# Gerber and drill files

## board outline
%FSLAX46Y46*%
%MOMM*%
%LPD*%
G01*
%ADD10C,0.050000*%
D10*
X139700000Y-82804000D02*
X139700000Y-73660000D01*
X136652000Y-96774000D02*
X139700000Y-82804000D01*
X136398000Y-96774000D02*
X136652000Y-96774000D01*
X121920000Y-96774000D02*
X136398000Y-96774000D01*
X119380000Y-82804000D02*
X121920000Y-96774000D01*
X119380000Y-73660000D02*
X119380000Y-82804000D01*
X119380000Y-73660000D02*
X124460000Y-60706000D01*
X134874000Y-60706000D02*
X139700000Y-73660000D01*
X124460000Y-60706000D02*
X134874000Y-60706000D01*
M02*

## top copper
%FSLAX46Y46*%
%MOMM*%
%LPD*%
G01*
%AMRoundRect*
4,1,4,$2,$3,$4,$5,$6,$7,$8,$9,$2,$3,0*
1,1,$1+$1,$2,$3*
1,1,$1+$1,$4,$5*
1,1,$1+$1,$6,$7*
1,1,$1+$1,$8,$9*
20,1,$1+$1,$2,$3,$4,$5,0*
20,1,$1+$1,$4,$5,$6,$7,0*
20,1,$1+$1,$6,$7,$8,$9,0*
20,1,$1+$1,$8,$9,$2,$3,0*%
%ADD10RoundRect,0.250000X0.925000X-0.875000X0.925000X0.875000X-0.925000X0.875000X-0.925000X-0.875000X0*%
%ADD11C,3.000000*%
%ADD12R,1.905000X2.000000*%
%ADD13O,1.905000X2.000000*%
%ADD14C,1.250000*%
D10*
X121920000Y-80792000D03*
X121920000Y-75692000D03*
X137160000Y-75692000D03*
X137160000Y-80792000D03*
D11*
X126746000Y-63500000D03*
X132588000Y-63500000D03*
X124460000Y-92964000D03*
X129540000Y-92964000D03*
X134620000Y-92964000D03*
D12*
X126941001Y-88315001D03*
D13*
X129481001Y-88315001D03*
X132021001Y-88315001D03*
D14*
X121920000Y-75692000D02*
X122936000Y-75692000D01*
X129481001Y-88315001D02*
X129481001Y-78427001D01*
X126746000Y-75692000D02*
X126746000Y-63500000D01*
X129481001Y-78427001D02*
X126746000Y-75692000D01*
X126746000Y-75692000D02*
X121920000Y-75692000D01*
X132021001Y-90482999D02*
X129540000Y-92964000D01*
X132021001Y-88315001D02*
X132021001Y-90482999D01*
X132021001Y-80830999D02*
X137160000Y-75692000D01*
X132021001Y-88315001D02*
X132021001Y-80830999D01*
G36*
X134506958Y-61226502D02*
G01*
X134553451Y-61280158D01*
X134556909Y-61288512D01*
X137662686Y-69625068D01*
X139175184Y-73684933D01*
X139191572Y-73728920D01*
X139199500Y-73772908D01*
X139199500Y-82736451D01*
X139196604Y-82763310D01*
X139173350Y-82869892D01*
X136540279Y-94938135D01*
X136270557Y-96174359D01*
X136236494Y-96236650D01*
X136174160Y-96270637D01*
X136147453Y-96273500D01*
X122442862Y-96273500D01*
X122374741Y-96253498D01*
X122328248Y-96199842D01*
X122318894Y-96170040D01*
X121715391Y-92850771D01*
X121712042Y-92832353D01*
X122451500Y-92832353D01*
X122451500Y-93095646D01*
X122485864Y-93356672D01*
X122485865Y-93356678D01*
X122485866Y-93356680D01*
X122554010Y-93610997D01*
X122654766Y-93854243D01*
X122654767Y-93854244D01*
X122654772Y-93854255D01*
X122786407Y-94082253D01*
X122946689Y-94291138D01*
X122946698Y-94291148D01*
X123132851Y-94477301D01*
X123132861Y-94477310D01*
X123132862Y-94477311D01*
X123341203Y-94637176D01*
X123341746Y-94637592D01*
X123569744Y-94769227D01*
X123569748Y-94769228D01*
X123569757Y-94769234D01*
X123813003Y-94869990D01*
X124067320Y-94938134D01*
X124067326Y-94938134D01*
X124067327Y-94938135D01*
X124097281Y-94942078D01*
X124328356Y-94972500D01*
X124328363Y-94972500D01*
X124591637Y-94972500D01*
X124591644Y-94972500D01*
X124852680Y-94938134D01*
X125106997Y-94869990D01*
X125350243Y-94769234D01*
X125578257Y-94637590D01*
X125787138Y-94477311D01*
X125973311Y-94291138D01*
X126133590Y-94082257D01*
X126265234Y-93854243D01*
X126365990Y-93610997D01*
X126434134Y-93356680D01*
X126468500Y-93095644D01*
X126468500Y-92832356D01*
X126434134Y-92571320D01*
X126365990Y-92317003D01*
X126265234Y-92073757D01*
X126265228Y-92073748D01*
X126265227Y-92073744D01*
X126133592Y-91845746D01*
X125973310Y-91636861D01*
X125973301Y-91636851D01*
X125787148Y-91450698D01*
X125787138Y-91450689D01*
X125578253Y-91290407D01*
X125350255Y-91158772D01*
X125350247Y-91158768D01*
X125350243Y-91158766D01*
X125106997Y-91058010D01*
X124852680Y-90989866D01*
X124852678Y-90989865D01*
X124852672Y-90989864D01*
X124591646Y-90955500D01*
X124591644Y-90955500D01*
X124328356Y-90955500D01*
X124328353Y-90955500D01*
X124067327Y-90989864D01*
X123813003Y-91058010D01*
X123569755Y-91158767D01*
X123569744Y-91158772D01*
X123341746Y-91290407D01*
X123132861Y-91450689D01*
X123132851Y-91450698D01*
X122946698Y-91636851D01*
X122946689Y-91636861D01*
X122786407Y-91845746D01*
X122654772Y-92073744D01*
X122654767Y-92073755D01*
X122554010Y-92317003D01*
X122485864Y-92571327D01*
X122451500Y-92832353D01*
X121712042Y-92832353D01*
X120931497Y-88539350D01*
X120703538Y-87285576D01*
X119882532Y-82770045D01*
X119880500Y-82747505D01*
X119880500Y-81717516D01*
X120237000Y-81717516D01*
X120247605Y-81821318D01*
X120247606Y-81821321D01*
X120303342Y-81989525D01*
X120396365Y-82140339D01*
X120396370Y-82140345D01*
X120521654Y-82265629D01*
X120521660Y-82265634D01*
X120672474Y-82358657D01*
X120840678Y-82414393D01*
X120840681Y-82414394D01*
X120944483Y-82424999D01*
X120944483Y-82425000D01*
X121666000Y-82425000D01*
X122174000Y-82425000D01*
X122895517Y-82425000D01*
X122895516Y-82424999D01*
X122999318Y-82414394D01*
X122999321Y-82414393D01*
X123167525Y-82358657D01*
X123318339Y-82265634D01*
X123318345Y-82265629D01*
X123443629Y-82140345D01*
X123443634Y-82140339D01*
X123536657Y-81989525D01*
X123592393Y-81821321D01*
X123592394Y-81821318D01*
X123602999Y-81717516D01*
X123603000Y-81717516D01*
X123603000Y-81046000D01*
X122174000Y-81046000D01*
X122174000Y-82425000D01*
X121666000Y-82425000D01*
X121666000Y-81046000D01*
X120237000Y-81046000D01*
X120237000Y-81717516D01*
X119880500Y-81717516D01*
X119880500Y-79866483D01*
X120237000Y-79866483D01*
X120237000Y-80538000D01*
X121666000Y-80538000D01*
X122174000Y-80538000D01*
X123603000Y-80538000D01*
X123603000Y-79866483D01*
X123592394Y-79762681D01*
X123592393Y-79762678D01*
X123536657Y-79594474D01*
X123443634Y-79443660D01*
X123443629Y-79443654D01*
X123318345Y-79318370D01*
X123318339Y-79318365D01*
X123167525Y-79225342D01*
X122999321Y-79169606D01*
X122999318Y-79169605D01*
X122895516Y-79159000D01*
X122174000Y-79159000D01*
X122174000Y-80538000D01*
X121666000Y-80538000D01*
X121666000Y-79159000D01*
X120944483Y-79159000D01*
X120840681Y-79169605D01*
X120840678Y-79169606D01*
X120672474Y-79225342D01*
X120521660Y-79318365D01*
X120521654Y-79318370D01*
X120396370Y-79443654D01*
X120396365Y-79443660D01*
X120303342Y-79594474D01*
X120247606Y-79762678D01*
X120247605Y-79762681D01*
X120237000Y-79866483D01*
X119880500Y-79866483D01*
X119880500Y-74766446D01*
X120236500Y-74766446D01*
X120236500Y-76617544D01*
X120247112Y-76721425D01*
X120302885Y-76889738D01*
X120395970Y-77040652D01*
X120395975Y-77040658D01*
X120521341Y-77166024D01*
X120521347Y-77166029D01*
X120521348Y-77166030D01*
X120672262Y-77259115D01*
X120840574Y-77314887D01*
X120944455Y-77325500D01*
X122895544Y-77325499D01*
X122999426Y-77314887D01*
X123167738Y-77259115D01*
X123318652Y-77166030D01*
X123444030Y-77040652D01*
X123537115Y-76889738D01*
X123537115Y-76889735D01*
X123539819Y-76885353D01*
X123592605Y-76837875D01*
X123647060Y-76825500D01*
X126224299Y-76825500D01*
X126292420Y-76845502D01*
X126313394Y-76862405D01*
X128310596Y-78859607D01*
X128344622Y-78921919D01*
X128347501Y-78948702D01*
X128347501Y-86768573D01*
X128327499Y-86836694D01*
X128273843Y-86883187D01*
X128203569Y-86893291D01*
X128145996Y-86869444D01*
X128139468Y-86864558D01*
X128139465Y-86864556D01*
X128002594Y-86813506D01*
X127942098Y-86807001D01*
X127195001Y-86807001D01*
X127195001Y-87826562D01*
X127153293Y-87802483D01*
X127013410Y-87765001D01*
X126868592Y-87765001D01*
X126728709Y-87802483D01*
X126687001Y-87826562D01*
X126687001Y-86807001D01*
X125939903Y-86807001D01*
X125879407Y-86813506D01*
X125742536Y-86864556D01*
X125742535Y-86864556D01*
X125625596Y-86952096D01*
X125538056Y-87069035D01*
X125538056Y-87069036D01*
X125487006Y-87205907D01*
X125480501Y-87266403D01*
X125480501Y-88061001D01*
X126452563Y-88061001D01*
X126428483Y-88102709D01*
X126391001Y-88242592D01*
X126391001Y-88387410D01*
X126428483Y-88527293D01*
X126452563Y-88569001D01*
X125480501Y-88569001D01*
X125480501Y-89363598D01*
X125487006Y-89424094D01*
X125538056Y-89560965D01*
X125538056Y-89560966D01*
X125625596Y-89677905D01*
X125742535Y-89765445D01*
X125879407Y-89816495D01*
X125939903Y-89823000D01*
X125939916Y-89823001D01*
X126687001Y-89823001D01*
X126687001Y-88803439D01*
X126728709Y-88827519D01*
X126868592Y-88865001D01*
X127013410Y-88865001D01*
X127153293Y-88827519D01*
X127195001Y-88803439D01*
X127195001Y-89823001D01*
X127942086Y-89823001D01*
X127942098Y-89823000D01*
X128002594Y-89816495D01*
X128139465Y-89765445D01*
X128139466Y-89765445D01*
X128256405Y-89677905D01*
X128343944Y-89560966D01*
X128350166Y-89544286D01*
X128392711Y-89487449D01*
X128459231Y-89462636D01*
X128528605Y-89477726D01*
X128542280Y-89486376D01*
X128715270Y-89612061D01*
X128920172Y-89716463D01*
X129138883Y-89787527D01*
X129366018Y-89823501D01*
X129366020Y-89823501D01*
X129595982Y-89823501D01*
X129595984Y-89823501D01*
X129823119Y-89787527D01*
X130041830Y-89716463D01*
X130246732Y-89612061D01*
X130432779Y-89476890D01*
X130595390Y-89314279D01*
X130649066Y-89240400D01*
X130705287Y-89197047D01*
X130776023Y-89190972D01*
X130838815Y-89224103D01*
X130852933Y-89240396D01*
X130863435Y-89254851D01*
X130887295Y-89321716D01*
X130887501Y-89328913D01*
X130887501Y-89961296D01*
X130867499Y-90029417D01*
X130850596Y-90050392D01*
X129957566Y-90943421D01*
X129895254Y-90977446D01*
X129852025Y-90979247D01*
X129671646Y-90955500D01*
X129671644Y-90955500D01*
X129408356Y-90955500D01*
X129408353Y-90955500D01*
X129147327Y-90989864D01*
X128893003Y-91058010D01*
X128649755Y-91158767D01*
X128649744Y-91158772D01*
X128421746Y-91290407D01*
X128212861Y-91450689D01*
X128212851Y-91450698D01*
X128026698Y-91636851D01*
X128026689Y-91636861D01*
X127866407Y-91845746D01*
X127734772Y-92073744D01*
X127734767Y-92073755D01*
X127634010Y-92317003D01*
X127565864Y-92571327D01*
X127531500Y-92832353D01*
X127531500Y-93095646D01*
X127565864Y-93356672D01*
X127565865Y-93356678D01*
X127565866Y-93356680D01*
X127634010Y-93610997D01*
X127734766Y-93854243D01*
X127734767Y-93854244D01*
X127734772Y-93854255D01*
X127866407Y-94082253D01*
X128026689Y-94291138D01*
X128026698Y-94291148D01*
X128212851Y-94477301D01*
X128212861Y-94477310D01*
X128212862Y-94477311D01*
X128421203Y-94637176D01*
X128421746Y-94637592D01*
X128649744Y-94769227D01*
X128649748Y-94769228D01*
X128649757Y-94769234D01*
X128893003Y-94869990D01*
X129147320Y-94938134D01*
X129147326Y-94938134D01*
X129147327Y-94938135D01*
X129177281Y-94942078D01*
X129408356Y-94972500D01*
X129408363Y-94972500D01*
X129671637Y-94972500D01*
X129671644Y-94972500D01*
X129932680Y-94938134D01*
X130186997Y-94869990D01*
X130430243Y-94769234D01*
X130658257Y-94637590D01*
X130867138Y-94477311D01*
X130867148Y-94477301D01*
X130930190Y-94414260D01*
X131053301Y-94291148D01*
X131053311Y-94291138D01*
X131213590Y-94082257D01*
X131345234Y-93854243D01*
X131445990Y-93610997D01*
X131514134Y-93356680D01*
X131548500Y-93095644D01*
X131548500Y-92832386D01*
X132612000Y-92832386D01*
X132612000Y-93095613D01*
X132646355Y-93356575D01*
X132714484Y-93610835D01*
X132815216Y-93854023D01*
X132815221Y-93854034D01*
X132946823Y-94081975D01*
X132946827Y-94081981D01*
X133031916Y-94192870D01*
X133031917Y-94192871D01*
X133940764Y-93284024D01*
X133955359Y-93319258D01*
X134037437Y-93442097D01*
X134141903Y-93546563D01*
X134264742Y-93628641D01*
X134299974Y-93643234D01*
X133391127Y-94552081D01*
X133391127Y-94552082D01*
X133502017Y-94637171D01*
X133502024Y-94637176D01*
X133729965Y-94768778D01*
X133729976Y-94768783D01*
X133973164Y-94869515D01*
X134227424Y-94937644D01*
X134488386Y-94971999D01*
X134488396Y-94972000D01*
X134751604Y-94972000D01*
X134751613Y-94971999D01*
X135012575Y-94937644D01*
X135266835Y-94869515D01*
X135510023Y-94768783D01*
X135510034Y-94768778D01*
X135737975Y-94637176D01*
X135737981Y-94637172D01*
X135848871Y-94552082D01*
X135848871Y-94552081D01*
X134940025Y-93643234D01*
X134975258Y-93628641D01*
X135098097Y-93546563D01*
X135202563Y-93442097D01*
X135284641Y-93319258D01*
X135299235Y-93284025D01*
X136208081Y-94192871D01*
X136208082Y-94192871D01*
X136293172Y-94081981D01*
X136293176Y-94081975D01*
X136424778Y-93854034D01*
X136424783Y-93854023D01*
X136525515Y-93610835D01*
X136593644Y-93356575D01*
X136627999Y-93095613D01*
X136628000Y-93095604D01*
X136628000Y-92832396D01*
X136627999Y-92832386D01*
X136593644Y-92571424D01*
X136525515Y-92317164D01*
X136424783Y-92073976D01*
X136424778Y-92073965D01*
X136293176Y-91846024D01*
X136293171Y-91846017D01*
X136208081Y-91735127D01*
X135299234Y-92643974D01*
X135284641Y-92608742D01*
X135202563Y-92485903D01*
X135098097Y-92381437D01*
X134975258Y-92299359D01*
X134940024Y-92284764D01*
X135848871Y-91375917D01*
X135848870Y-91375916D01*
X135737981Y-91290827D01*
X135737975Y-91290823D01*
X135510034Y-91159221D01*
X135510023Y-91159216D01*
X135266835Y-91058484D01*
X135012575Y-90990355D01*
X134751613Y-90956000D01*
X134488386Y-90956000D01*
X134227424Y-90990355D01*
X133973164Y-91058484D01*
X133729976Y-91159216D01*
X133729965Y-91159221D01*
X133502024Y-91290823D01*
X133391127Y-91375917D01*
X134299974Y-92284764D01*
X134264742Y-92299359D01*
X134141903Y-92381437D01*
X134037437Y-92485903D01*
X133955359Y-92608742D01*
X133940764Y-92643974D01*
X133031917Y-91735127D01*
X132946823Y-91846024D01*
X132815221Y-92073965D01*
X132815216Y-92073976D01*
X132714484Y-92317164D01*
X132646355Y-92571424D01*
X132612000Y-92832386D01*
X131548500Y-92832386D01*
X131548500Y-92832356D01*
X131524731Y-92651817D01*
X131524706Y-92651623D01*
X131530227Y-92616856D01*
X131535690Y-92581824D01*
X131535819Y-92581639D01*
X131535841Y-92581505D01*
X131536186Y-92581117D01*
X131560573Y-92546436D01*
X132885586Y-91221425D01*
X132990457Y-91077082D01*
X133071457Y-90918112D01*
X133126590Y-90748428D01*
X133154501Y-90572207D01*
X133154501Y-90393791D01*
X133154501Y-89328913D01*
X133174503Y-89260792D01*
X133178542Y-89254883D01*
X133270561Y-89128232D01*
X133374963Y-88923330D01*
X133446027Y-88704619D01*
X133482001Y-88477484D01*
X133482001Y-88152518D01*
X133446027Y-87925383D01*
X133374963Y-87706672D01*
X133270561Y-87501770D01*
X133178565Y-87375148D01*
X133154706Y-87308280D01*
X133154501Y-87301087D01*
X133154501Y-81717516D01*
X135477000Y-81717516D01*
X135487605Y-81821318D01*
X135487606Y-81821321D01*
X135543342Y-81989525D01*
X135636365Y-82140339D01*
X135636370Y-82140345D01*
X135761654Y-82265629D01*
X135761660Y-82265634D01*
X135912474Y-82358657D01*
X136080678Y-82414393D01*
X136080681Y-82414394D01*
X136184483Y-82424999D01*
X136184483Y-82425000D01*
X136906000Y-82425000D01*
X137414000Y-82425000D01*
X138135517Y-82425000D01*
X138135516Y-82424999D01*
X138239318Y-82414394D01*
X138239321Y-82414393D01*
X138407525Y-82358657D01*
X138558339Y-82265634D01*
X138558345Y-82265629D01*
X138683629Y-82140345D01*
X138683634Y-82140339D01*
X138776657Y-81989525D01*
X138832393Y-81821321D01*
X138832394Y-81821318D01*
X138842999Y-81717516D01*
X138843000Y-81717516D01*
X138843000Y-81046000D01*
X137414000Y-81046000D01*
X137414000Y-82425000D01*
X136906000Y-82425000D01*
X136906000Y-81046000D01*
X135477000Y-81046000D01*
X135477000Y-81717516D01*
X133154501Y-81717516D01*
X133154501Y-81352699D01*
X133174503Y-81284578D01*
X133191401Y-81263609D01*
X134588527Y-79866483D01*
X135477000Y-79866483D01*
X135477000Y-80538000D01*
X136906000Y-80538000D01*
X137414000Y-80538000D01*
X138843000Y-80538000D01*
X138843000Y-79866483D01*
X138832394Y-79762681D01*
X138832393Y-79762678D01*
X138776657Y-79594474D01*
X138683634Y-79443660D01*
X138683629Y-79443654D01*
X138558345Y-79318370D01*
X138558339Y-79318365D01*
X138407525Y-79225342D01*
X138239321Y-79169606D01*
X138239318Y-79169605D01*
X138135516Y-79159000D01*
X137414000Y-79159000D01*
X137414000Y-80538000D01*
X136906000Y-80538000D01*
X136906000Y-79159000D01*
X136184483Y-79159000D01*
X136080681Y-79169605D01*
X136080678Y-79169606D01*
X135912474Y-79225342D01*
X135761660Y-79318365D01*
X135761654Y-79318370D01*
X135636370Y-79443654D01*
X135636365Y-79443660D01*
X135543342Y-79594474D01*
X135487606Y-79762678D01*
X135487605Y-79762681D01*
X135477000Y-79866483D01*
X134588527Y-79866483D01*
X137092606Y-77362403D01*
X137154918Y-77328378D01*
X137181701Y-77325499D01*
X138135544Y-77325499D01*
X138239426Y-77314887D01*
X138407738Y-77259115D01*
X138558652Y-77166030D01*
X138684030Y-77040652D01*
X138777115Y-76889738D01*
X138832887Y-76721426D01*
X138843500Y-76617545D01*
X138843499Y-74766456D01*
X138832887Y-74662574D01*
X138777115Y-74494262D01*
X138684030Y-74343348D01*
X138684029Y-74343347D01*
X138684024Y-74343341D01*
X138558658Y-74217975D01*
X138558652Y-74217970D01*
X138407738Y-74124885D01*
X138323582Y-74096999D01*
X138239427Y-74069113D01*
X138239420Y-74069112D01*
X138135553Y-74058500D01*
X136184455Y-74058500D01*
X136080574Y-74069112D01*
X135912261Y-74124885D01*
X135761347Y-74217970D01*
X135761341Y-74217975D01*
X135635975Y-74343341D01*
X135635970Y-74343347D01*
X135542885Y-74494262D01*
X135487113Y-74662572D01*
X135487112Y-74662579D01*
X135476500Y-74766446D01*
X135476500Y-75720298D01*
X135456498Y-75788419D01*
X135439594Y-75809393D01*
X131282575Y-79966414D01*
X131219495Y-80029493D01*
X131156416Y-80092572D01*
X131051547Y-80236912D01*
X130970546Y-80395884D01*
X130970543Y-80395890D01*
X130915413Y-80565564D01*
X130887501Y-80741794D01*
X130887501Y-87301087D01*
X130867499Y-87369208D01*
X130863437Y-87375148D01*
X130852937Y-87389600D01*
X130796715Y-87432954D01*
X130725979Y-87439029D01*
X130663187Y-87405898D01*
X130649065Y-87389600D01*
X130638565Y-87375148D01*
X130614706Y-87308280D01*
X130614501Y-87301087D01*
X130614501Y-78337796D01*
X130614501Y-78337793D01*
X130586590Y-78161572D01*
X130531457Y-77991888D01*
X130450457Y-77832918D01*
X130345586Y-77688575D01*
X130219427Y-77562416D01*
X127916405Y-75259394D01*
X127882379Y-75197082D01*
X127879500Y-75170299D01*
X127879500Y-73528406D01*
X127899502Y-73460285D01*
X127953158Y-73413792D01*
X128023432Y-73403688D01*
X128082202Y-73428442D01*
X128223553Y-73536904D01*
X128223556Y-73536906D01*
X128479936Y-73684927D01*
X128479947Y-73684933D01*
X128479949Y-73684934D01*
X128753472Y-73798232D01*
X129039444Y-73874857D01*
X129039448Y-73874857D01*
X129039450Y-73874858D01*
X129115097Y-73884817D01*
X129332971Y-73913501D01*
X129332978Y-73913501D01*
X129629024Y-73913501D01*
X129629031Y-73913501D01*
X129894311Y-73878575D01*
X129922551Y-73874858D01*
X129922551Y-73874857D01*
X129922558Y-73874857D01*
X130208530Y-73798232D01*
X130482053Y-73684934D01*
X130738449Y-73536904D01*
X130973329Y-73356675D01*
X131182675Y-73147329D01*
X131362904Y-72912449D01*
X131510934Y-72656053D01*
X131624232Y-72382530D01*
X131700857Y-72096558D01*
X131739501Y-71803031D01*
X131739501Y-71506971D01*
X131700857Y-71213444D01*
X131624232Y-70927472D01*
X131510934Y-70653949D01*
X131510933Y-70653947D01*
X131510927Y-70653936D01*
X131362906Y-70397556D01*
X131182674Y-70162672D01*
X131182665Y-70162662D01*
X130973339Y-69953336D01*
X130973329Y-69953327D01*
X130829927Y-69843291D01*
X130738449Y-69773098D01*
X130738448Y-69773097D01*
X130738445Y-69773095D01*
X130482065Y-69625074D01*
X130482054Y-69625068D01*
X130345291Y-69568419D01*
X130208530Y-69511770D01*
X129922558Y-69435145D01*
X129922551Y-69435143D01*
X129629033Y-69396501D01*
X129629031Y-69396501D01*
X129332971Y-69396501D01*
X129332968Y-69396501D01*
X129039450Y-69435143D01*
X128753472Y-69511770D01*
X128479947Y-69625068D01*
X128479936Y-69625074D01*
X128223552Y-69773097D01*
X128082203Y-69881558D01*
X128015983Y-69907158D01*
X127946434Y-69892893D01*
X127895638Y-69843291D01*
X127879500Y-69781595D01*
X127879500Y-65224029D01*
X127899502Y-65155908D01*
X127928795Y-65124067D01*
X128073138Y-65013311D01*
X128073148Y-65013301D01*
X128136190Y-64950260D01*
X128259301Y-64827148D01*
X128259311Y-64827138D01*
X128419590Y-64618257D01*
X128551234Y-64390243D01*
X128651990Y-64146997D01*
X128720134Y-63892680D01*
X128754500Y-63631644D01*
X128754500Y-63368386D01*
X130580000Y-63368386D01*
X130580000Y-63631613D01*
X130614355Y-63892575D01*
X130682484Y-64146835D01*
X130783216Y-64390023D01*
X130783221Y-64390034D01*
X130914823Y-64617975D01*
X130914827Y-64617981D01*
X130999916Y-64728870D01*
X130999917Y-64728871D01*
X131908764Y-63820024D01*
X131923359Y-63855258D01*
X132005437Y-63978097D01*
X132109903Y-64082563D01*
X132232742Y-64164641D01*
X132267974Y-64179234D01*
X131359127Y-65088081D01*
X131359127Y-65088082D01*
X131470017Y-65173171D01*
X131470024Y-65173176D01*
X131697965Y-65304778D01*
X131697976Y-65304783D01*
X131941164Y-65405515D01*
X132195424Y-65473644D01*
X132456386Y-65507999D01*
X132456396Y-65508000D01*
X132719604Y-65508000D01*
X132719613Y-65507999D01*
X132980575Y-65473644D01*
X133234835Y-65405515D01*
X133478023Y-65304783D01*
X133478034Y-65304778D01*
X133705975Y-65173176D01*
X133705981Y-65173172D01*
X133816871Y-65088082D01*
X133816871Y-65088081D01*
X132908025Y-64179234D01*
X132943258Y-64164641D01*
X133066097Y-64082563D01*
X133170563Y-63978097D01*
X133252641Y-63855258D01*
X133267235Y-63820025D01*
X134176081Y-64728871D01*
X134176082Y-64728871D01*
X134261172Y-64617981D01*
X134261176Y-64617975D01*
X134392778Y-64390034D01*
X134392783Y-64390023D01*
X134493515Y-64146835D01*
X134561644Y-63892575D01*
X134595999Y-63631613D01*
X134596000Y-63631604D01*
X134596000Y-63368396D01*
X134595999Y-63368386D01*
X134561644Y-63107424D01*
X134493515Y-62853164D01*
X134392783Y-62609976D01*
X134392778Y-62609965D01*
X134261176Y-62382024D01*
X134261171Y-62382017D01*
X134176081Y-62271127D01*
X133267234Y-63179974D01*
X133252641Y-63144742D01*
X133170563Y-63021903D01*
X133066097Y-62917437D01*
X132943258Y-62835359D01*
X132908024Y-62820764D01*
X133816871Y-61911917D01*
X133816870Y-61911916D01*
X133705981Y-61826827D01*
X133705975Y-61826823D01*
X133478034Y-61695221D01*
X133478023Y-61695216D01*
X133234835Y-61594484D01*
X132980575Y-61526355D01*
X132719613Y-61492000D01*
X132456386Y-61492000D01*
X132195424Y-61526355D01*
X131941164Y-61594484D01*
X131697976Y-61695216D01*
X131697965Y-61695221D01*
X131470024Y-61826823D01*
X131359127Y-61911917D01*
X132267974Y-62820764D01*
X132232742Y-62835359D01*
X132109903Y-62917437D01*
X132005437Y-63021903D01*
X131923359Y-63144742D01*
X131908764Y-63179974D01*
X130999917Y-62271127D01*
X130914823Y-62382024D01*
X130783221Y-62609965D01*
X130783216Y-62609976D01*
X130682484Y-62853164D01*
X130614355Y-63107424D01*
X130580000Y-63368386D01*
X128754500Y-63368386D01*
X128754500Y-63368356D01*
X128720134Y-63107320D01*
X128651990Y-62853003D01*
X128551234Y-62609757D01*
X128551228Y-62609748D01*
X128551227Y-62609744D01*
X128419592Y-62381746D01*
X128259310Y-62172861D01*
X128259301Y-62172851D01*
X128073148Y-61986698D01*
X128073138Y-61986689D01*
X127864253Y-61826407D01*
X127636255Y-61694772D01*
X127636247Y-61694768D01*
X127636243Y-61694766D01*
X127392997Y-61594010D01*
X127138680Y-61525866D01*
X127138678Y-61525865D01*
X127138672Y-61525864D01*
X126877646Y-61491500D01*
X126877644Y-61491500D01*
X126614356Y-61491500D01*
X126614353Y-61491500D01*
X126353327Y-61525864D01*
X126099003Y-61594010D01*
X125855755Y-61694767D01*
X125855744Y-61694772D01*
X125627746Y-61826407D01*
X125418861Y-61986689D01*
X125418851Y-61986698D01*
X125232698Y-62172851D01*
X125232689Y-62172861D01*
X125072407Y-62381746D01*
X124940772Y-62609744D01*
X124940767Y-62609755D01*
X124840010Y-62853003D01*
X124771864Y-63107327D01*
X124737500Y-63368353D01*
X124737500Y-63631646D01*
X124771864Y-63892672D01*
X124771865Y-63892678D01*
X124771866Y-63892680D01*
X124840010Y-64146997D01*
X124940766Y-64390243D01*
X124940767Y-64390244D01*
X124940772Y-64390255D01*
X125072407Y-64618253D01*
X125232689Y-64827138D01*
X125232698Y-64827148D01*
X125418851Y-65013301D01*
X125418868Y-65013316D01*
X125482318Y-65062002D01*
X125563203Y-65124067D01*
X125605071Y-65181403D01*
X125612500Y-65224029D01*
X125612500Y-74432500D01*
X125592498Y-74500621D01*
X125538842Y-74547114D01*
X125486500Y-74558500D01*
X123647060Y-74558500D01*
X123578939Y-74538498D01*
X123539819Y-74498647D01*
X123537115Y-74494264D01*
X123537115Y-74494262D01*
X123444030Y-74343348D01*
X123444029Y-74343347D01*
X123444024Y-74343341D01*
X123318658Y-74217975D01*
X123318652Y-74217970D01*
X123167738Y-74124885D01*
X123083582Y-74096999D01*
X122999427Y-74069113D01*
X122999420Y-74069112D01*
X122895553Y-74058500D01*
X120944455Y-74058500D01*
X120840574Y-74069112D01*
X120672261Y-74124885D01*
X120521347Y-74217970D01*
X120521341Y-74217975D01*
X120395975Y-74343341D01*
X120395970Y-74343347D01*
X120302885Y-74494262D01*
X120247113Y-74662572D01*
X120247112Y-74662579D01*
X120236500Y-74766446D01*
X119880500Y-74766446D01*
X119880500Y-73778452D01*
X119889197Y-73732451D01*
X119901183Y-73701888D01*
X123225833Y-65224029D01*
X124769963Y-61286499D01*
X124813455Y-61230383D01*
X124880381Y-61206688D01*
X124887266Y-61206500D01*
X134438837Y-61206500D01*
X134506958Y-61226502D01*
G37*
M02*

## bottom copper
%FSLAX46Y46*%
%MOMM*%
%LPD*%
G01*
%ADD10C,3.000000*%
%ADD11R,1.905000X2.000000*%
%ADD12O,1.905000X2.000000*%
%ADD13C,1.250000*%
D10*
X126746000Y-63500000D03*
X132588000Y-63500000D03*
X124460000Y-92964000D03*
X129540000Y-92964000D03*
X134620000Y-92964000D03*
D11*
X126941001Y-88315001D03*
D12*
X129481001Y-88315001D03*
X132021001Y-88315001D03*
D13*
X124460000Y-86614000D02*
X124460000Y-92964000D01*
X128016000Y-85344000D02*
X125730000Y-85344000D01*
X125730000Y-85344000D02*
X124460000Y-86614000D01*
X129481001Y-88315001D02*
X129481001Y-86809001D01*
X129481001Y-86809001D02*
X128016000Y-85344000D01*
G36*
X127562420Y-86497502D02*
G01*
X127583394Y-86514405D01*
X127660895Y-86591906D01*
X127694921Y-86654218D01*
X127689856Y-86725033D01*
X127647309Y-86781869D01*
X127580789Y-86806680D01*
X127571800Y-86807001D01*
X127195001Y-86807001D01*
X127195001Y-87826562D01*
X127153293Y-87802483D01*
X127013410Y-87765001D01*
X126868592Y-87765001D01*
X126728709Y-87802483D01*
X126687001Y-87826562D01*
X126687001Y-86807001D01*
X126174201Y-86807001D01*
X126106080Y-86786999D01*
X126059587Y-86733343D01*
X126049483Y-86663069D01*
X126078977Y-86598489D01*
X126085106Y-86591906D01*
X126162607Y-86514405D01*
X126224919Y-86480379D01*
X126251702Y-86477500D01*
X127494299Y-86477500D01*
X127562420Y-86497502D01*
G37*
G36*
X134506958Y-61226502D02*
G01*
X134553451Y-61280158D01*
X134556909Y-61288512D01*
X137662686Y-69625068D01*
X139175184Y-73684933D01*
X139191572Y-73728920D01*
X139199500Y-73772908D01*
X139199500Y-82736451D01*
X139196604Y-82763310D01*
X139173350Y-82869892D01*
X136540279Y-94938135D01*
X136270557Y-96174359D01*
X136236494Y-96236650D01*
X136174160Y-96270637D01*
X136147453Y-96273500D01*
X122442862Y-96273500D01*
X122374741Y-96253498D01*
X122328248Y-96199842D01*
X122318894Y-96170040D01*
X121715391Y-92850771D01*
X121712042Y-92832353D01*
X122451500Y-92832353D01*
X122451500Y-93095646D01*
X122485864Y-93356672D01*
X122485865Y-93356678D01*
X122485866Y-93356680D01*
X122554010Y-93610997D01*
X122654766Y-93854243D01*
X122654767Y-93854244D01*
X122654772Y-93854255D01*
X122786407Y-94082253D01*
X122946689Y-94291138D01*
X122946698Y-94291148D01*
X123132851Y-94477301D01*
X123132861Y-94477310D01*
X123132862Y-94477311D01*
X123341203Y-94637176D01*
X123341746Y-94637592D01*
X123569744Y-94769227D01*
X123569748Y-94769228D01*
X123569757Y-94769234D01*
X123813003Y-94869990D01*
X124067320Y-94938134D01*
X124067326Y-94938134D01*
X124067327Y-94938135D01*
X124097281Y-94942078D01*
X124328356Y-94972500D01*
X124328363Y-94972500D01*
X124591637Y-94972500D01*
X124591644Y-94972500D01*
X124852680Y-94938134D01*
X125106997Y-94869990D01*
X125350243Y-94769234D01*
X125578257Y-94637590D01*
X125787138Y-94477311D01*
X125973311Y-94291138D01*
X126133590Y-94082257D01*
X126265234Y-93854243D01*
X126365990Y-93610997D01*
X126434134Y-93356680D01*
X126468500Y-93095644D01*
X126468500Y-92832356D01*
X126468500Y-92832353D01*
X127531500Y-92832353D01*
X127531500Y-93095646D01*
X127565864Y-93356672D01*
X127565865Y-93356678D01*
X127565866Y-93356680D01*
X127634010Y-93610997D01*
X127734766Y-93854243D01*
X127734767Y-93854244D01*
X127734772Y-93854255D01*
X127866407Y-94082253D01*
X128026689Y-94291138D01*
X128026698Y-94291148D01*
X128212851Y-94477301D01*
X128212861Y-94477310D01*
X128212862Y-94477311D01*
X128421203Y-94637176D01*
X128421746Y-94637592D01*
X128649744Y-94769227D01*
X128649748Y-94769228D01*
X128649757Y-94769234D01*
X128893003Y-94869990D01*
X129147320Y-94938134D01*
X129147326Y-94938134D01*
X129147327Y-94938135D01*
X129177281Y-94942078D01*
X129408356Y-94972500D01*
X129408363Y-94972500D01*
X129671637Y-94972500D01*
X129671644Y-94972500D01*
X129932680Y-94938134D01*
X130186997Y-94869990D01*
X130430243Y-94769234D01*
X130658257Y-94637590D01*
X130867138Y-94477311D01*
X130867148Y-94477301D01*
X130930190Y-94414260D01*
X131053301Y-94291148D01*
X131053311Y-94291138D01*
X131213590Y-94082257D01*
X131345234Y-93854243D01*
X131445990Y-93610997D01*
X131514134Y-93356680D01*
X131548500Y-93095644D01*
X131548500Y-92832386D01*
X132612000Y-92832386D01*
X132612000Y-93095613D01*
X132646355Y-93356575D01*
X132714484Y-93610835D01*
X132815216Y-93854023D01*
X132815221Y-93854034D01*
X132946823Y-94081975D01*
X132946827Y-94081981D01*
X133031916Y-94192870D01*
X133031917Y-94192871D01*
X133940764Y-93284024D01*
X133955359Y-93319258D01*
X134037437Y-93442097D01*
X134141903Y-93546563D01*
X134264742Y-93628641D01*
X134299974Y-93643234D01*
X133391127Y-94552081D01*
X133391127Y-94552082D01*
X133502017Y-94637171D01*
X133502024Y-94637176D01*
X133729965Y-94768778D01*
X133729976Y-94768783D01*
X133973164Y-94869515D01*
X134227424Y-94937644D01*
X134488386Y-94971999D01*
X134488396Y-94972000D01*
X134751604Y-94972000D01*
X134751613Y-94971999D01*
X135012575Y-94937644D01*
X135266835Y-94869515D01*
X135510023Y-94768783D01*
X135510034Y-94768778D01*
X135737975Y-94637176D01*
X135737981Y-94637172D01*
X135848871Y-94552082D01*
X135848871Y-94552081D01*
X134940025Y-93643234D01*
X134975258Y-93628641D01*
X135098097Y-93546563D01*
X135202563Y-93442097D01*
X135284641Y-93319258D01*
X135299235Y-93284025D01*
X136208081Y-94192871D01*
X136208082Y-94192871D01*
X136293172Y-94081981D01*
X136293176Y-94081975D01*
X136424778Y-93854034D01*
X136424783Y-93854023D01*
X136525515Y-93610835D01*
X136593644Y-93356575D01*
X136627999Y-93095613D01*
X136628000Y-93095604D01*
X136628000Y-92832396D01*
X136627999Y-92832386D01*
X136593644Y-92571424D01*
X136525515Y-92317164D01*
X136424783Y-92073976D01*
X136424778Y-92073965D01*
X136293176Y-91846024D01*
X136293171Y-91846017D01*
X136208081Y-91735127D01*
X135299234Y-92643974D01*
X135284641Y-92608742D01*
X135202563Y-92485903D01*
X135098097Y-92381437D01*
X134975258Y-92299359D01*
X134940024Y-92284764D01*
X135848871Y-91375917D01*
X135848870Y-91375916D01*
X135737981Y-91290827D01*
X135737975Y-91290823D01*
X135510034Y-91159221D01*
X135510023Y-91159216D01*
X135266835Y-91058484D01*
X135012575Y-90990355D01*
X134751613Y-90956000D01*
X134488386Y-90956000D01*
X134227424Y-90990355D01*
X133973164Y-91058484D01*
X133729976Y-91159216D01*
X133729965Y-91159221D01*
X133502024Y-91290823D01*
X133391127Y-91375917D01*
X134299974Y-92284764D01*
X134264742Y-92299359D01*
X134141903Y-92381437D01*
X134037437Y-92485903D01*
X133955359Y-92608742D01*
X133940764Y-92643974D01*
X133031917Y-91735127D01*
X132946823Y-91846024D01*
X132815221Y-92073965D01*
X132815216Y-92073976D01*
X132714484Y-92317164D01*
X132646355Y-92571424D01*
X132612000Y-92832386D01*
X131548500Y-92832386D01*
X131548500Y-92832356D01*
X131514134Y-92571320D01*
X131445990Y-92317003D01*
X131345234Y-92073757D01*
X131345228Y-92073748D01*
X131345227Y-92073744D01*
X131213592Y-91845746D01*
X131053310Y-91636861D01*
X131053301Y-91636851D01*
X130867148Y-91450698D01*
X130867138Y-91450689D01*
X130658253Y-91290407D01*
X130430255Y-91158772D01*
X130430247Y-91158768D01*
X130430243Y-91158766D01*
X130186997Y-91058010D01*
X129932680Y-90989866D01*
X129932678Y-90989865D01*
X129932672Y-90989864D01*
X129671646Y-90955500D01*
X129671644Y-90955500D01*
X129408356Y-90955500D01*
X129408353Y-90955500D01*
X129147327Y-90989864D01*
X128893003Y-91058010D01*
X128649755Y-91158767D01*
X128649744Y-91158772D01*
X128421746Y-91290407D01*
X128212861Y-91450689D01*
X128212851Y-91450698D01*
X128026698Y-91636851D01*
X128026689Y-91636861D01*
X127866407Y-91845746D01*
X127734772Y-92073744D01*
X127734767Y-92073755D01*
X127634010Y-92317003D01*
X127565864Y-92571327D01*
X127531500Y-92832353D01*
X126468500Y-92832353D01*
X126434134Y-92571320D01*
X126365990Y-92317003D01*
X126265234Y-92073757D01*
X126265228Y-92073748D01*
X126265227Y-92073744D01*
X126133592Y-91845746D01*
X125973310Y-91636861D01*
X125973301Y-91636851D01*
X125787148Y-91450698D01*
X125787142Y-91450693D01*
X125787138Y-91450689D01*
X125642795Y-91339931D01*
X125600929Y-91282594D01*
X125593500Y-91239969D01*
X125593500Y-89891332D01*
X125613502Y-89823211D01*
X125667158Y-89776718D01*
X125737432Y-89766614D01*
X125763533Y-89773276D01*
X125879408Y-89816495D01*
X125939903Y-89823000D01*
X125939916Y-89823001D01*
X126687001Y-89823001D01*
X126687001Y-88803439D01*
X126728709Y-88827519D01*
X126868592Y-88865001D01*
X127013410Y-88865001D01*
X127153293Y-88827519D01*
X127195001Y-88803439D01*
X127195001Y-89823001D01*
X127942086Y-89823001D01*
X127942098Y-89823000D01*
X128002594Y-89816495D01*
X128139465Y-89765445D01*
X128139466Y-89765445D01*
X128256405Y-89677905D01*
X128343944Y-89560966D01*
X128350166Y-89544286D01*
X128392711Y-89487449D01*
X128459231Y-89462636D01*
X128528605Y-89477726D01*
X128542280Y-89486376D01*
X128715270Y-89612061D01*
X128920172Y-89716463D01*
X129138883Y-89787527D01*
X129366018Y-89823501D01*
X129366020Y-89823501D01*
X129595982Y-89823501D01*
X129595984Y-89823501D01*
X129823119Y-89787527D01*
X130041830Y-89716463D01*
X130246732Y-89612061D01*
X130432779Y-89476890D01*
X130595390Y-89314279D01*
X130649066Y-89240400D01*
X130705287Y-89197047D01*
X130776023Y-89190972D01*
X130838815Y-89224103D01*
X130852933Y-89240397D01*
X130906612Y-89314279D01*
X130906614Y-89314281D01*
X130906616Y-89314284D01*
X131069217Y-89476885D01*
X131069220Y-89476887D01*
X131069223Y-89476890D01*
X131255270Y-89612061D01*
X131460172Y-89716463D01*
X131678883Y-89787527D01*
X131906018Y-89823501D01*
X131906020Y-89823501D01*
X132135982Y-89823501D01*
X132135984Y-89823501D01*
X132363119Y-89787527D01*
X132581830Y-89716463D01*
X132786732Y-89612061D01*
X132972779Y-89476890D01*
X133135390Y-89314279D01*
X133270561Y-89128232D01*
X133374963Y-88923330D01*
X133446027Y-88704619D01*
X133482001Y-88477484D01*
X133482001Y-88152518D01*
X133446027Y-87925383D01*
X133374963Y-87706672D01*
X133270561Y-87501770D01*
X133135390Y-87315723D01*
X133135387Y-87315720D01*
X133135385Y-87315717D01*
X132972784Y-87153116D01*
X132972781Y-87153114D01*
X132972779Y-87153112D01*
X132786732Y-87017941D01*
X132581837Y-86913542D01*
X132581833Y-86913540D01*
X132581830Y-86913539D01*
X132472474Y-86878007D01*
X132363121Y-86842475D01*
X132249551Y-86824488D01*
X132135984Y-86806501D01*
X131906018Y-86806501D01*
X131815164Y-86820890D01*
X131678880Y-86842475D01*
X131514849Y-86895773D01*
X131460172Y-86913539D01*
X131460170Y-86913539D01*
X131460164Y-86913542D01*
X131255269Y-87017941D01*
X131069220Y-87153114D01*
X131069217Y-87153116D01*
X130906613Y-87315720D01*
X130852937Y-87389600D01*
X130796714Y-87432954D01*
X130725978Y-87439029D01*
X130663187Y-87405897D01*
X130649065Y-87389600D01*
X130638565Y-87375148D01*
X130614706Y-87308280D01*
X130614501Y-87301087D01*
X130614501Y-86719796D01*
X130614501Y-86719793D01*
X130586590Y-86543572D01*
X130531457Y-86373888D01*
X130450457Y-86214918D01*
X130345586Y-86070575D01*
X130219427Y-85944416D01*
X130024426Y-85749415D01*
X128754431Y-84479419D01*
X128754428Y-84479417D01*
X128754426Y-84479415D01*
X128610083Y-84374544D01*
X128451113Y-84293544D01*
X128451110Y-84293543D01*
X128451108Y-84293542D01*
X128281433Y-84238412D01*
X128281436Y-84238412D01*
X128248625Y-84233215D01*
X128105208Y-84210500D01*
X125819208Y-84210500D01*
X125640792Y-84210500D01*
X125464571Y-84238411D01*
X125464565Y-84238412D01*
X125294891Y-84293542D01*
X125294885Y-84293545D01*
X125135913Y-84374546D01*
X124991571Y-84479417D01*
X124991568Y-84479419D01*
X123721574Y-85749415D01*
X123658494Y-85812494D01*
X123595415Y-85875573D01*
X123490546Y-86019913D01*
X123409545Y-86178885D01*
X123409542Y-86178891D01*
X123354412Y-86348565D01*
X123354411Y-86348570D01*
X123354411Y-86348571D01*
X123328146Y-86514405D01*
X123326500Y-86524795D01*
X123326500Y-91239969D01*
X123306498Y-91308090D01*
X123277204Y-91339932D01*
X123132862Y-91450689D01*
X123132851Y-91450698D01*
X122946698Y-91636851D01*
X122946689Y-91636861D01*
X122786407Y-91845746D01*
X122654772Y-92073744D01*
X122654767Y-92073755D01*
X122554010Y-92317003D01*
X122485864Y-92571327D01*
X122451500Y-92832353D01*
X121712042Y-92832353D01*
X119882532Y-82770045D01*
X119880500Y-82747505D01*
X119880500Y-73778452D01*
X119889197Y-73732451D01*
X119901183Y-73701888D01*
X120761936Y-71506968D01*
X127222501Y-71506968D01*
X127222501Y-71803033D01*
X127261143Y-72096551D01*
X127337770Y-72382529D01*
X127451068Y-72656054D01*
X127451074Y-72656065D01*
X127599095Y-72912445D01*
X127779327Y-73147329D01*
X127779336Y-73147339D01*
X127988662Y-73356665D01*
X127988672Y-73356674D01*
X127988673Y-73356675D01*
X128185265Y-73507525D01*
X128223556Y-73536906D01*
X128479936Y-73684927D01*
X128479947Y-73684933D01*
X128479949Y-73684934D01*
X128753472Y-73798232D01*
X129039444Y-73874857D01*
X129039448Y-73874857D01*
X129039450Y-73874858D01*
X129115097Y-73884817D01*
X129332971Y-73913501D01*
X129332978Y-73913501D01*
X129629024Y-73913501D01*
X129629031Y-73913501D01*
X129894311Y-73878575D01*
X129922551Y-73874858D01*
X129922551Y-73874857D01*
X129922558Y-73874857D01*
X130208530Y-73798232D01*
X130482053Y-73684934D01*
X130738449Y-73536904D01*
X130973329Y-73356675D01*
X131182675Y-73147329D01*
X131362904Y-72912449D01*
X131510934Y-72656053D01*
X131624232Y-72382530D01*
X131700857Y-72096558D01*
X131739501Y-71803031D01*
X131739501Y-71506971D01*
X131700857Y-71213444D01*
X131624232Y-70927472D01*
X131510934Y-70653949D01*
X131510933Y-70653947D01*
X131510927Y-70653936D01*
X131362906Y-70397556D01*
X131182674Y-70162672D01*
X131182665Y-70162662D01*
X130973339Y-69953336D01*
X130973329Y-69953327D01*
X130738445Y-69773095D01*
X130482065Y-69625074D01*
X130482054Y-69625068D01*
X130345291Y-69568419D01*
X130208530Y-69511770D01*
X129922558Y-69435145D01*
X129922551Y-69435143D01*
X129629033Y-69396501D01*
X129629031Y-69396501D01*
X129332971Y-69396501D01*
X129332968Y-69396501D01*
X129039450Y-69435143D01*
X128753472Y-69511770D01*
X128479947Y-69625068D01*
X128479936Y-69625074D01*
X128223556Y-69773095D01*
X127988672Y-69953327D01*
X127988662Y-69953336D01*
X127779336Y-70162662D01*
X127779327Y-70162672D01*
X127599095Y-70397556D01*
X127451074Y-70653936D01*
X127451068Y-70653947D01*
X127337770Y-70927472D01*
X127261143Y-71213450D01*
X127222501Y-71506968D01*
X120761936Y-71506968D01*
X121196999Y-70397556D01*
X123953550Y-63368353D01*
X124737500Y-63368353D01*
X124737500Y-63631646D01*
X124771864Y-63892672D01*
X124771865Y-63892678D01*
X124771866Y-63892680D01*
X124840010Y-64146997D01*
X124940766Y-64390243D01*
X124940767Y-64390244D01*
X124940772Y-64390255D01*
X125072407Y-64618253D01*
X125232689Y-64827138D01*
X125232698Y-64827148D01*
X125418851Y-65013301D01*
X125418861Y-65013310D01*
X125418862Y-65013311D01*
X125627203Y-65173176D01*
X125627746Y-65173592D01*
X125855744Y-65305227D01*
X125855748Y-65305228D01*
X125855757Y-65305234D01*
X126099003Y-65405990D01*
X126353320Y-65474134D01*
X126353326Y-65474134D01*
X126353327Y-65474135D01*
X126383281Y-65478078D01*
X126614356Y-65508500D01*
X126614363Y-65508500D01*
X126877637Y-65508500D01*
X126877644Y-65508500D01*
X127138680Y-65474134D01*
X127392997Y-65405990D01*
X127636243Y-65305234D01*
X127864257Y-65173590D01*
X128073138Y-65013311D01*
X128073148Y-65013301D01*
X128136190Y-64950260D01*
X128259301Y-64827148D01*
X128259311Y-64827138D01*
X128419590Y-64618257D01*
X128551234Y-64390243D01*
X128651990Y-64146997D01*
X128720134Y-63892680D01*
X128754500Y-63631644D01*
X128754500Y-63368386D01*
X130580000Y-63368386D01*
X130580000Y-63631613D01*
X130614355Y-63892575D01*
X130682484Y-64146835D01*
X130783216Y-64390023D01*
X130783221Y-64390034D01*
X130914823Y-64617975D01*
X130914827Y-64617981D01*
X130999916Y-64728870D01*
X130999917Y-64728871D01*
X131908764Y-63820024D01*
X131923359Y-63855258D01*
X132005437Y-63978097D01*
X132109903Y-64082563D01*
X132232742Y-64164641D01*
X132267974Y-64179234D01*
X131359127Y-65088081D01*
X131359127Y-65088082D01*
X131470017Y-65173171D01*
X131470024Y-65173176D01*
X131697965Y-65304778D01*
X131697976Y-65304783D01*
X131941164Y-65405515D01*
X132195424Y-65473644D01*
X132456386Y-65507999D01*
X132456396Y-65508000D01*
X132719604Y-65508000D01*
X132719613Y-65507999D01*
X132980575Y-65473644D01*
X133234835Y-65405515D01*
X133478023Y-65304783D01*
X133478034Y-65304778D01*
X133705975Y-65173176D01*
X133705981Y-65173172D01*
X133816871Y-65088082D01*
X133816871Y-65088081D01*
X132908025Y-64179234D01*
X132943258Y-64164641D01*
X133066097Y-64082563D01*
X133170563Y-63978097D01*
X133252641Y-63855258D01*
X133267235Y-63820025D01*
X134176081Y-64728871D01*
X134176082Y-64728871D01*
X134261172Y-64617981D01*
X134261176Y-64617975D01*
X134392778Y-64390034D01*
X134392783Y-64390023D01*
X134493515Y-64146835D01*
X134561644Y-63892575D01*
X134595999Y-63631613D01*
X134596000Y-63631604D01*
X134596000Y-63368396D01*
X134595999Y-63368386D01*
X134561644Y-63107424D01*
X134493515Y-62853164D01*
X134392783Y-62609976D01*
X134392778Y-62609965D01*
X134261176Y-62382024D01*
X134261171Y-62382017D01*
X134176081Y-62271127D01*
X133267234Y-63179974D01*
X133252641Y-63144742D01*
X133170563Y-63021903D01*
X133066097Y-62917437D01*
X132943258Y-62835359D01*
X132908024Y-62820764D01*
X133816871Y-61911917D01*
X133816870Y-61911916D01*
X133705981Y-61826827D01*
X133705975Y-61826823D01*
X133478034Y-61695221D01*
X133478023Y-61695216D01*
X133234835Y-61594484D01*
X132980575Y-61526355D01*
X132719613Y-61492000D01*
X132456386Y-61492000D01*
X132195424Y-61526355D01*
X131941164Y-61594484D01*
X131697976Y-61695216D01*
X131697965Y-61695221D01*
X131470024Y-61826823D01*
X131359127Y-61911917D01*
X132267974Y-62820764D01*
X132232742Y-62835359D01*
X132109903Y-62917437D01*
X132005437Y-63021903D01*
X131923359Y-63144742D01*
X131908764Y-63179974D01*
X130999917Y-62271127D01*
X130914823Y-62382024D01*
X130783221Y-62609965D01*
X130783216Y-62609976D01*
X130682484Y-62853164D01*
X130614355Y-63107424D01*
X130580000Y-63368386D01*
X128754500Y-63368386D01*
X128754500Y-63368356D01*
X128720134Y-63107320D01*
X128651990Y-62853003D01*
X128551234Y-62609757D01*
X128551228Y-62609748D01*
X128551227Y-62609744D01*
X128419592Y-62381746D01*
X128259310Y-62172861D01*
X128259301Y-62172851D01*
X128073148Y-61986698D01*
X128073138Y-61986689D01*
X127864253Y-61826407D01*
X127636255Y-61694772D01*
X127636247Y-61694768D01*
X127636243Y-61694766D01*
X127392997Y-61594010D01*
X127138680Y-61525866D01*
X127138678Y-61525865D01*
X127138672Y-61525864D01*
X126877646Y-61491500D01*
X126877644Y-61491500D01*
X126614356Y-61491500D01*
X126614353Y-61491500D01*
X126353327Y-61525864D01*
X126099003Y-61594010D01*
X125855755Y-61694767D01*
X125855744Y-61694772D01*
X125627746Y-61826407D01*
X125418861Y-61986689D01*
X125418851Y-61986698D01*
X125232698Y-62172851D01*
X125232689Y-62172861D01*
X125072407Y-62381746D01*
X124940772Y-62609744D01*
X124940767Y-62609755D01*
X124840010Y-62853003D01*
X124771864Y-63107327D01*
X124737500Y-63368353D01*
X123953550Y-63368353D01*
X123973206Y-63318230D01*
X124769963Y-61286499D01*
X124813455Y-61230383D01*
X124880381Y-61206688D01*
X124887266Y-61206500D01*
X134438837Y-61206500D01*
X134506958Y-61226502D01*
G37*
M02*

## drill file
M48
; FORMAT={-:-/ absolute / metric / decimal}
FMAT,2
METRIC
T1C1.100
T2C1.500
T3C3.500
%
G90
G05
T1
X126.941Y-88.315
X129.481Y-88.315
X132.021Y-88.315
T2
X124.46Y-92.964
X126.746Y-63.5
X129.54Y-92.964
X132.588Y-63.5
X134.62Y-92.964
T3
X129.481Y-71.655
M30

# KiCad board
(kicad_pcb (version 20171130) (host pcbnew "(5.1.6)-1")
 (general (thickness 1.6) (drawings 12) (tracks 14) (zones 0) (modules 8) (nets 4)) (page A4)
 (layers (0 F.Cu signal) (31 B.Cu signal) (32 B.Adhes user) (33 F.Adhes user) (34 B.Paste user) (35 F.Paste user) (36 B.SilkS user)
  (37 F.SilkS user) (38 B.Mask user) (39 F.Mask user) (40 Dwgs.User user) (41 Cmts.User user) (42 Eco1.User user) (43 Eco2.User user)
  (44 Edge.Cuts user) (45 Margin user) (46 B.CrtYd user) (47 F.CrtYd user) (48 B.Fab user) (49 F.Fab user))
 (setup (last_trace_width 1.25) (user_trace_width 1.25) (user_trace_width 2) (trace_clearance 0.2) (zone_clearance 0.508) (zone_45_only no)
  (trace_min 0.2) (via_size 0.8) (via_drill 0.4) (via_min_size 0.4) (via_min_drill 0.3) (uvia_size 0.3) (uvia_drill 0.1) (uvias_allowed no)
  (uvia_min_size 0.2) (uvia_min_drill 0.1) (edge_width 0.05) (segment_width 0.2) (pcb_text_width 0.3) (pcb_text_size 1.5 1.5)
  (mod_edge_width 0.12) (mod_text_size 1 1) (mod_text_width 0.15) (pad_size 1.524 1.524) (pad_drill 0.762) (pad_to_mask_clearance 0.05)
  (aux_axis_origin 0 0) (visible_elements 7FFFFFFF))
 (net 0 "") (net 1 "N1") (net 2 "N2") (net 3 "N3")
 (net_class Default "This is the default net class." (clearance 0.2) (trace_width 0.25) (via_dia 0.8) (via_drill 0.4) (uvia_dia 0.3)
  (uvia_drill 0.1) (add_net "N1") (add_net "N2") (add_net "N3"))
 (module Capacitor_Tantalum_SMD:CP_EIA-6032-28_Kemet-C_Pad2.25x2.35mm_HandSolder (layer F.Cu) (at 121.92 78.242 90)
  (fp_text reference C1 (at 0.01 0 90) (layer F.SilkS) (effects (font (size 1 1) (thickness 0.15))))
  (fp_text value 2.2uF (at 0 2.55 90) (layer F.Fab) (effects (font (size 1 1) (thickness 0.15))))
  (pad 1 smd roundrect (at -2.55 0 90) (size 2.25 2.35) (layers F.Cu F.Paste F.Mask) (roundrect_rratio 0.111111) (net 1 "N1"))
  (pad 2 smd roundrect (at 2.55 0 90) (size 2.25 2.35) (layers F.Cu F.Paste F.Mask) (roundrect_rratio 0.111111) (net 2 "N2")))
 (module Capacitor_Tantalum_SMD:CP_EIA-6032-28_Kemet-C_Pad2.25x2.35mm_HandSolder (layer F.Cu) (at 137.16 78.242 90)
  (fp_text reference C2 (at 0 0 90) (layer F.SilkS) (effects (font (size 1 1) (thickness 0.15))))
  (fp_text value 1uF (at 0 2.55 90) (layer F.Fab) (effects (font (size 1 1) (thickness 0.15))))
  (pad 2 smd roundrect (at 2.55 0 90) (size 2.25 2.35) (layers F.Cu F.Paste F.Mask) (roundrect_rratio 0.111111) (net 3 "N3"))
  (pad 1 smd roundrect (at -2.55 0 90) (size 2.25 2.35) (layers F.Cu F.Paste F.Mask) (roundrect_rratio 0.111111) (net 1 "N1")))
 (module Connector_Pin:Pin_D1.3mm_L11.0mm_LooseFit (layer F.Cu) (at 126.746 63.5)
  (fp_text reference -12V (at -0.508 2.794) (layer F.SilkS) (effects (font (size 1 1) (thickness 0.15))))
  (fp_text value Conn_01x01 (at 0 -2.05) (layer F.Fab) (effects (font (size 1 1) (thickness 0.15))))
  (pad 1 thru_hole circle (at 0 0) (size 3 3) (drill 1.5) (layers *.Cu *.Mask) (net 2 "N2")))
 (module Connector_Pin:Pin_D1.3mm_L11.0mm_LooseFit (layer F.Cu) (at 132.588 63.5)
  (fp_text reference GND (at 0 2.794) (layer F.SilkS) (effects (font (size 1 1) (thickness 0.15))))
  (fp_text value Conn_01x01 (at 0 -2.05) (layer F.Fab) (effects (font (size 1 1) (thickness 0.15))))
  (pad 1 thru_hole circle (at 0 0) (size 3 3) (drill 1.5) (layers *.Cu *.Mask) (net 1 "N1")))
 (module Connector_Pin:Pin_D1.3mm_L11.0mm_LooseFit (layer F.Cu) (at 124.46 92.964)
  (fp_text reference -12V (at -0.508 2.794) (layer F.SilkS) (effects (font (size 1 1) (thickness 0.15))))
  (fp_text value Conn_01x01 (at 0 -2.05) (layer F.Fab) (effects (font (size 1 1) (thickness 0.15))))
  (pad 1 thru_hole circle (at 0 0) (size 3 3) (drill 1.5) (layers *.Cu *.Mask) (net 2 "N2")))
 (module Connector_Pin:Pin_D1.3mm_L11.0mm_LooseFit (layer F.Cu) (at 129.54 92.964)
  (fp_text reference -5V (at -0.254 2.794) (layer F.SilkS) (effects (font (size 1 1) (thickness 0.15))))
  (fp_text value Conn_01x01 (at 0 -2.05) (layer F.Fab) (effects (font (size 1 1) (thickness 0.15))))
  (pad 1 thru_hole circle (at 0 0) (size 3 3) (drill 1.5) (layers *.Cu *.Mask) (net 3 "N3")))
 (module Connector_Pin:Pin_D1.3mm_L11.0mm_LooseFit (layer F.Cu) (at 134.62 92.964)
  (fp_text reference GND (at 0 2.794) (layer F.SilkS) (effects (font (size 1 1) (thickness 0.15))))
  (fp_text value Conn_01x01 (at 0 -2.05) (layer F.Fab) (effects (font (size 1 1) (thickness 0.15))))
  (pad 1 thru_hole circle (at 0 0) (size 3 3) (drill 1.5) (layers *.Cu *.Mask) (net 1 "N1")))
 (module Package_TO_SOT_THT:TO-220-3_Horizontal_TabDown (layer F.Cu) (at 126.941001 88.315001)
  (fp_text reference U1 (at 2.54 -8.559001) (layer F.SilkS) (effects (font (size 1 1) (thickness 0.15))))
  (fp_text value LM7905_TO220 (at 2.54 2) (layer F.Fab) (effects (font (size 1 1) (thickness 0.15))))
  (pad "" np_thru_hole oval (at 2.54 -16.66) (size 3.5 3.5) (drill 3.5) (layers *.Cu *.Mask))
  (pad 1 thru_hole rect (at 0 0) (size 1.905 2) (drill 1.1) (layers *.Cu *.Mask) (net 1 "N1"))
  (pad 2 thru_hole oval (at 2.54 0) (size 1.905 2) (drill 1.1) (layers *.Cu *.Mask) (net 2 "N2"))
  (pad 3 thru_hole oval (at 5.08 0) (size 1.905 2) (drill 1.1) (layers *.Cu *.Mask) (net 3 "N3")))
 (gr_line (start 139.7 82.804) (end 139.7 73.66) (layer Edge.Cuts) (width 0.05))
 (gr_line (start 136.652 96.774) (end 139.7 82.804) (layer Edge.Cuts) (width 0.05))
 (gr_line (start 136.398 96.774) (end 136.652 96.774) (layer Edge.Cuts) (width 0.05))
 (gr_line (start 121.92 96.774) (end 136.398 96.774) (layer Edge.Cuts) (width 0.05))
 (gr_line (start 119.38 82.804) (end 121.92 96.774) (layer Edge.Cuts) (width 0.05))
 (gr_line (start 119.38 73.66) (end 119.38 82.804) (layer Edge.Cuts) (width 0.05))
 (gr_line (start 119.38 73.66) (end 124.46 60.706) (layer Edge.Cuts) (width 0.05))
 (gr_line (start 134.874 60.706) (end 139.7 73.66) (layer Edge.Cuts) (width 0.05))
 (gr_line (start 124.46 60.706) (end 134.874 60.706) (layer Edge.Cuts) (width 0.05))
 (segment (start 121.92 75.692) (end 122.936 75.692) (width 1.25) (layer F.Cu) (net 2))
 (segment (start 129.481001 88.315001) (end 129.481001 78.427001) (width 1.25) (layer F.Cu) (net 2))
 (segment (start 126.746 75.692) (end 126.746 63.5) (width 1.25) (layer F.Cu) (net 2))
 (segment (start 129.481001 78.427001) (end 126.746 75.692) (width 1.25) (layer F.Cu) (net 2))
 (segment (start 126.746 75.692) (end 121.92 75.692) (width 1.25) (layer F.Cu) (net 2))
 (segment (start 124.46 86.614) (end 124.46 92.964) (width 1.25) (layer B.Cu) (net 2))
 (segment (start 128.016 85.344) (end 125.73 85.344) (width 1.25) (layer B.Cu) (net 2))
 (segment (start 125.73 85.344) (end 124.46 86.614) (width 1.25) (layer B.Cu) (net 2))
 (segment (start 129.481001 88.315001) (end 129.481001 86.809001) (width 1.25) (layer B.Cu) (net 2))
 (segment (start 129.481001 86.809001) (end 128.016 85.344) (width 1.25) (layer B.Cu) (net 2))
 (segment (start 132.021001 90.482999) (end 129.54 92.964) (width 1.25) (layer F.Cu) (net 3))
 (segment (start 132.021001 88.315001) (end 132.021001 90.482999) (width 1.25) (layer F.Cu) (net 3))
 (segment (start 132.021001 80.830999) (end 137.16 75.692) (width 1.25) (layer F.Cu) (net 3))
 (segment (start 132.021001 88.315001) (end 132.021001 80.830999) (width 1.25) (layer F.Cu) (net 3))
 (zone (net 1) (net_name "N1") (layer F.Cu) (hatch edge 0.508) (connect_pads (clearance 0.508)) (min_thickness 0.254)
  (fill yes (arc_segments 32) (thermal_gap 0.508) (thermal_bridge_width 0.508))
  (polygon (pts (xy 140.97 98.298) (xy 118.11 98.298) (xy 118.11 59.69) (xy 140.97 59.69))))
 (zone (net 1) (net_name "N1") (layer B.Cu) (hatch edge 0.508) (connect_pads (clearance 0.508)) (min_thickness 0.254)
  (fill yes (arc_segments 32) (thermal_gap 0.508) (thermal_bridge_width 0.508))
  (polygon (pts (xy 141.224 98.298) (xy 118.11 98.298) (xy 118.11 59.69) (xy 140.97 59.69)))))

